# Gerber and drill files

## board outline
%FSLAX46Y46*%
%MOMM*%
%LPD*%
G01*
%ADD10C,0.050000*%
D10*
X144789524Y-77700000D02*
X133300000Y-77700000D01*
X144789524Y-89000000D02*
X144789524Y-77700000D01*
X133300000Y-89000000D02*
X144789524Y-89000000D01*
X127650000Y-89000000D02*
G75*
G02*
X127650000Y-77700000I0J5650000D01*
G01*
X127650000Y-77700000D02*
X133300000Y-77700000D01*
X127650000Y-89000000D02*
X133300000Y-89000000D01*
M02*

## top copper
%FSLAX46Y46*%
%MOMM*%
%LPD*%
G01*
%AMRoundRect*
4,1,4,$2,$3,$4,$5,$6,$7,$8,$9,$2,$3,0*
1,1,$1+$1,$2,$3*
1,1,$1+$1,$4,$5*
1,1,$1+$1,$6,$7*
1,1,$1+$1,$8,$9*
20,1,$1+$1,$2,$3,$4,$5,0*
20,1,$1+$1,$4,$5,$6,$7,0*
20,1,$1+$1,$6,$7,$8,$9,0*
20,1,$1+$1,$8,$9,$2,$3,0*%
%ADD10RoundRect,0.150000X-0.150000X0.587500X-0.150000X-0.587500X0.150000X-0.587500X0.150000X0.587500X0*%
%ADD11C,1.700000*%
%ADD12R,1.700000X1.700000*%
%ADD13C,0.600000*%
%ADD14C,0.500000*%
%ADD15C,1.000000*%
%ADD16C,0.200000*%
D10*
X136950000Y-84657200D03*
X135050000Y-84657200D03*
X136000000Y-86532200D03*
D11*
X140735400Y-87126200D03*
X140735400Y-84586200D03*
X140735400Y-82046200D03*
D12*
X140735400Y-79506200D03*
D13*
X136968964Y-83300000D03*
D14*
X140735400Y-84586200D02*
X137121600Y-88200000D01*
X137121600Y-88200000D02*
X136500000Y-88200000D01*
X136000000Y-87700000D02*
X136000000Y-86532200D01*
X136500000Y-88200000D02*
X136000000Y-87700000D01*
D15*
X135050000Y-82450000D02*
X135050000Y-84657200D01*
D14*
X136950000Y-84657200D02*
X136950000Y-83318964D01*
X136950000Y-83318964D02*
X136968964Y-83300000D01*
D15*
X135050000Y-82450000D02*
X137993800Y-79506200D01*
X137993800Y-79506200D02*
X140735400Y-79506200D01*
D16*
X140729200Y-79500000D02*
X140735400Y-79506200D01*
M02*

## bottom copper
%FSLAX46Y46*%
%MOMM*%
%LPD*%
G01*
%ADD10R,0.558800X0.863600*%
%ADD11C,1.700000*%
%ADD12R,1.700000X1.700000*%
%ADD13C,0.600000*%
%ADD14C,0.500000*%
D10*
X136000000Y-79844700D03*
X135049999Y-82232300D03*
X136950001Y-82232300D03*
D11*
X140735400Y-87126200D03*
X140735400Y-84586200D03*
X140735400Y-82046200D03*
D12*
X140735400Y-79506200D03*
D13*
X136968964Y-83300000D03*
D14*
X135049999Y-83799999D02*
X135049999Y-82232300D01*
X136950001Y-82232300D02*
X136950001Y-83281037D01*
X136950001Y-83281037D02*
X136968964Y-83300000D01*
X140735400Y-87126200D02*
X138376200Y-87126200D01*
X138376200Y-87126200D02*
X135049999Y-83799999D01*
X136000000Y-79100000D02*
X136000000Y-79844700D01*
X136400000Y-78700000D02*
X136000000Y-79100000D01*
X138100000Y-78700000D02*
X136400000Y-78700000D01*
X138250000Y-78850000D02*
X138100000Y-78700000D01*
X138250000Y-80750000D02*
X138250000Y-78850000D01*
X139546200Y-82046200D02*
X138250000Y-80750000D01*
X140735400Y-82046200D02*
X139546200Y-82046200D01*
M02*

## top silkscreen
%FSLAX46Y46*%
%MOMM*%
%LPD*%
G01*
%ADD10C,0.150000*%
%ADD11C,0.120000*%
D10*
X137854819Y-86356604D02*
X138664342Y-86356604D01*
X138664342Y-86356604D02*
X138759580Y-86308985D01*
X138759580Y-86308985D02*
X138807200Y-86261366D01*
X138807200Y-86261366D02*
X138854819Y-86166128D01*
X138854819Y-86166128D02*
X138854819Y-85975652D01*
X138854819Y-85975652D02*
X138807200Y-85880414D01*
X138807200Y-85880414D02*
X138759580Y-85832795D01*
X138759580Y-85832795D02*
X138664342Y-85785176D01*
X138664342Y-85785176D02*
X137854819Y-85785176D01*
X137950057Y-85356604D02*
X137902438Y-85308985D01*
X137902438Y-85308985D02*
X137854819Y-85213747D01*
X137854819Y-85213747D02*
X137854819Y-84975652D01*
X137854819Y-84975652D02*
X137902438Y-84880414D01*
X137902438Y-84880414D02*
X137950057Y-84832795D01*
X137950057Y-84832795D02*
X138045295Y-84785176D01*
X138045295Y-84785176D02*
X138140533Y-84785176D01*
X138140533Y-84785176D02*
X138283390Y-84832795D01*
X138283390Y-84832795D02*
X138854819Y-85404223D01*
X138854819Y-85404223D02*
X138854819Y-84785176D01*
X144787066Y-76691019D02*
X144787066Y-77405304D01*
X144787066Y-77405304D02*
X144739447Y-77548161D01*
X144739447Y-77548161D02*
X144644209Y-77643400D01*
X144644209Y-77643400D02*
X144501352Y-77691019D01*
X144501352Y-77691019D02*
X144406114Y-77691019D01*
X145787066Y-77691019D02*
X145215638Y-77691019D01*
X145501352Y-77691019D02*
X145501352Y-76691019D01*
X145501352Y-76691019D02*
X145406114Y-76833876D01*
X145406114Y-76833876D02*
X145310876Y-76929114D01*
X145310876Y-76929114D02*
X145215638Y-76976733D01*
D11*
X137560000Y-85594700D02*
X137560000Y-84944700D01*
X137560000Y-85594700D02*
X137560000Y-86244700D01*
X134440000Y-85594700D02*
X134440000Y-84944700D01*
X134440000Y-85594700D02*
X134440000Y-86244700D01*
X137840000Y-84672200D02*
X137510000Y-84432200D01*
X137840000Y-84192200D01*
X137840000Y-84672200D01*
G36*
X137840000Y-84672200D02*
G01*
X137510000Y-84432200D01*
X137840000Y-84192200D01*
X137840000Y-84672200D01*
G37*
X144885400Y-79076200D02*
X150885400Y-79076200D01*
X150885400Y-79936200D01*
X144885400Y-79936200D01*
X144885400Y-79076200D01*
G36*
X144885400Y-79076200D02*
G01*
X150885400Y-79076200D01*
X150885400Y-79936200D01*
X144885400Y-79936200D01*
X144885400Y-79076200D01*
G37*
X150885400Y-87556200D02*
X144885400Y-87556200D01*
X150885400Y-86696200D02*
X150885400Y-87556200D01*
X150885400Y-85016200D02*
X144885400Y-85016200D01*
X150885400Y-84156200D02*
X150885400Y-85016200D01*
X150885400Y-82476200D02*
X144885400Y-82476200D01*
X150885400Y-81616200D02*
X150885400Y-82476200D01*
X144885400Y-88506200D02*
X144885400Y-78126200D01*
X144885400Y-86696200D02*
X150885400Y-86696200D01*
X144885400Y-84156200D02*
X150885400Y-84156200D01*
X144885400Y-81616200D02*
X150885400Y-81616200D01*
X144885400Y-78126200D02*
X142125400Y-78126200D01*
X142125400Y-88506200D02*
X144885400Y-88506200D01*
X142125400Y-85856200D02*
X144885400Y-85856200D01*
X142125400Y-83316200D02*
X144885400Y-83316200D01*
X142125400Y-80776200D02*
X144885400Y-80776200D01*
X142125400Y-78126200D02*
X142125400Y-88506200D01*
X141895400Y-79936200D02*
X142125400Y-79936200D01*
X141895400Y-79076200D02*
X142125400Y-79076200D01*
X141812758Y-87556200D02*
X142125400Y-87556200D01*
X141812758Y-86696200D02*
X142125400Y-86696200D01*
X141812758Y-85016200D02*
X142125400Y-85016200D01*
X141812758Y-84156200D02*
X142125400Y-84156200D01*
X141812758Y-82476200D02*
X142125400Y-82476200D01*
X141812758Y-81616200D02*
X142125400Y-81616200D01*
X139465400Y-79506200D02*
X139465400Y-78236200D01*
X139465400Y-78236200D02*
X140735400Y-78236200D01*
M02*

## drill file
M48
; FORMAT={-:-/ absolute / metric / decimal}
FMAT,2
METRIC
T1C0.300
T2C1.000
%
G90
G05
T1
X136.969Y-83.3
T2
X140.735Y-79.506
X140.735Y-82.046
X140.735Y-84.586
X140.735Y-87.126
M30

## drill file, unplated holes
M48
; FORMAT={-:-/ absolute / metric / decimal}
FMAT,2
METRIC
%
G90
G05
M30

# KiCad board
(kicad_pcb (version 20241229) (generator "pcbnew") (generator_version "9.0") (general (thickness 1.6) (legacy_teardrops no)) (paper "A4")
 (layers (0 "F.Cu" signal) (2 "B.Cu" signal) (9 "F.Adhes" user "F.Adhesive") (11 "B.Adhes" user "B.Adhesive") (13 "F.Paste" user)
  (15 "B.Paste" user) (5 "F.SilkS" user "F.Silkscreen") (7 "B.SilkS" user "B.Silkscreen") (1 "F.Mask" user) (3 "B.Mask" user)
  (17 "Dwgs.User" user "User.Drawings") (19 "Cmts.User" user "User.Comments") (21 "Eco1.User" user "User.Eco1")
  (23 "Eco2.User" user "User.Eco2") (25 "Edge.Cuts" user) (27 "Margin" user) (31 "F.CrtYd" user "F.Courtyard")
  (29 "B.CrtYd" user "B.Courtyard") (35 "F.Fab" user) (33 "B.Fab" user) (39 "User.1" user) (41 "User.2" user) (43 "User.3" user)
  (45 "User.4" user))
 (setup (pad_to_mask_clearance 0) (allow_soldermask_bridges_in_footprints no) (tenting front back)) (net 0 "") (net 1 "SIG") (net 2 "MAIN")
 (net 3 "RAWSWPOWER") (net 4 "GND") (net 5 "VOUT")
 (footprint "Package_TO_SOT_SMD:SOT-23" (layer "F.Cu") (at 136 85.5947 -90)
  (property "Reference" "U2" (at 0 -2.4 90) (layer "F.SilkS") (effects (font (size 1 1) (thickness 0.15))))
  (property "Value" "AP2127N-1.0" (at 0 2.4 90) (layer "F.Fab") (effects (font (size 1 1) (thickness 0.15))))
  (fp_line (start 0 1.56) (end -0.65 1.56) (stroke (width 0.12) (type solid)) (layer "F.SilkS"))
  (fp_line (start 0 1.56) (end 0.65 1.56) (stroke (width 0.12) (type solid)) (layer "F.SilkS"))
  (fp_line (start 0 -1.56) (end -0.65 -1.56) (stroke (width 0.12) (type solid)) (layer "F.SilkS"))
  (fp_line (start 0 -1.56) (end 0.65 -1.56) (stroke (width 0.12) (type solid)) (layer "F.SilkS"))
  (fp_poly (pts (xy -1.1625 -1.51) (xy -1.4025 -1.84) (xy -0.9225 -1.84)) (stroke (width 0.12) (type solid)) (fill yes) (layer "F.SilkS"))
  (pad "1" smd roundrect (at -0.9375 -0.95 270) (size 1.475 0.6) (layers "F.Cu" "F.Mask" "F.Paste") (roundrect_rratio 0.25) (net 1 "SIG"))
  (pad "2" smd roundrect (at -0.9375 0.95 270) (size 1.475 0.6) (layers "F.Cu" "F.Mask" "F.Paste") (roundrect_rratio 0.25) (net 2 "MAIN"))
  (pad "3" smd roundrect (at 0.9375 0 270) (size 1.475 0.6) (layers "F.Cu" "F.Mask" "F.Paste") (roundrect_rratio 0.25) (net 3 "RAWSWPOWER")))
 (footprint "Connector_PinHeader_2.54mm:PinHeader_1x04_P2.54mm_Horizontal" (layer "F.Cu") (at 140.7354 79.5062)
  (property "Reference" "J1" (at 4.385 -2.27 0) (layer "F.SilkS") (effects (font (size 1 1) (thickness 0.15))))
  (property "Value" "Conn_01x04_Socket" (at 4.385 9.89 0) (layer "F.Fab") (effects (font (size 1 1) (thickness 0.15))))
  (fp_line (start -1.27 -1.27) (end 0 -1.27) (stroke (width 0.12) (type solid)) (layer "F.SilkS"))
  (fp_line (start -1.27 0) (end -1.27 -1.27) (stroke (width 0.12) (type solid)) (layer "F.SilkS"))
  (fp_line (start 1.077358 2.11) (end 1.39 2.11) (stroke (width 0.12) (type solid)) (layer "F.SilkS"))
  (fp_line (start 1.077358 2.97) (end 1.39 2.97) (stroke (width 0.12) (type solid)) (layer "F.SilkS"))
  (fp_line (start 1.077358 4.65) (end 1.39 4.65) (stroke (width 0.12) (type solid)) (layer "F.SilkS"))
  (fp_line (start 1.077358 5.51) (end 1.39 5.51) (stroke (width 0.12) (type solid)) (layer "F.SilkS"))
  (fp_line (start 1.077358 7.19) (end 1.39 7.19) (stroke (width 0.12) (type solid)) (layer "F.SilkS"))
  (fp_line (start 1.077358 8.05) (end 1.39 8.05) (stroke (width 0.12) (type solid)) (layer "F.SilkS"))
  (fp_line (start 1.16 -0.43) (end 1.39 -0.43) (stroke (width 0.12) (type solid)) (layer "F.SilkS"))
  (fp_line (start 1.16 0.43) (end 1.39 0.43) (stroke (width 0.12) (type solid)) (layer "F.SilkS"))
  (fp_line (start 1.39 -1.38) (end 1.39 9) (stroke (width 0.12) (type solid)) (layer "F.SilkS"))
  (fp_line (start 1.39 1.27) (end 4.15 1.27) (stroke (width 0.12) (type solid)) (layer "F.SilkS"))
  (fp_line (start 1.39 3.81) (end 4.15 3.81) (stroke (width 0.12) (type solid)) (layer "F.SilkS"))
  (fp_line (start 1.39 6.35) (end 4.15 6.35) (stroke (width 0.12) (type solid)) (layer "F.SilkS"))
  (fp_line (start 1.39 9) (end 4.15 9) (stroke (width 0.12) (type solid)) (layer "F.SilkS"))
  (fp_line (start 4.15 -1.38) (end 1.39 -1.38) (stroke (width 0.12) (type solid)) (layer "F.SilkS"))
  (fp_line (start 4.15 2.11) (end 10.15 2.11) (stroke (width 0.12) (type solid)) (layer "F.SilkS"))
  (fp_line (start 4.15 4.65) (end 10.15 4.65) (stroke (width 0.12) (type solid)) (layer "F.SilkS"))
  (fp_line (start 4.15 7.19) (end 10.15 7.19) (stroke (width 0.12) (type solid)) (layer "F.SilkS"))
  (fp_line (start 4.15 9) (end 4.15 -1.38) (stroke (width 0.12) (type solid)) (layer "F.SilkS"))
  (fp_line (start 10.15 2.11) (end 10.15 2.97) (stroke (width 0.12) (type solid)) (layer "F.SilkS"))
  (fp_line (start 10.15 2.97) (end 4.15 2.97) (stroke (width 0.12) (type solid)) (layer "F.SilkS"))
  (fp_line (start 10.15 4.65) (end 10.15 5.51) (stroke (width 0.12) (type solid)) (layer "F.SilkS"))
  (fp_line (start 10.15 5.51) (end 4.15 5.51) (stroke (width 0.12) (type solid)) (layer "F.SilkS"))
  (fp_line (start 10.15 7.19) (end 10.15 8.05) (stroke (width 0.12) (type solid)) (layer "F.SilkS"))
  (fp_line (start 10.15 8.05) (end 4.15 8.05) (stroke (width 0.12) (type solid)) (layer "F.SilkS"))
  (fp_rect (start 4.15 -0.43) (end 10.15 0.43) (stroke (width 0.12) (type solid)) (fill yes) (layer "F.SilkS"))
  (pad "1" thru_hole rect (at 0 0) (size 1.7 1.7) (drill 1) (layers "*.Cu" "*.Mask") (remove_unused_layers no) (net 2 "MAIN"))
  (pad "2" thru_hole circle (at 0 2.54) (size 1.7 1.7) (drill 1) (layers "*.Cu" "*.Mask") (remove_unused_layers no) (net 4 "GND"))
  (pad "3" thru_hole circle (at 0 5.08) (size 1.7 1.7) (drill 1) (layers "*.Cu" "*.Mask") (remove_unused_layers no) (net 3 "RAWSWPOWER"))
  (pad "4" thru_hole circle (at 0 7.62) (size 1.7 1.7) (drill 1) (layers "*.Cu" "*.Mask") (remove_unused_layers no) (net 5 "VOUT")))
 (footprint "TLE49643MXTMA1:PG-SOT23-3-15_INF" (layer "B.Cu") (at 136 81.0385 90)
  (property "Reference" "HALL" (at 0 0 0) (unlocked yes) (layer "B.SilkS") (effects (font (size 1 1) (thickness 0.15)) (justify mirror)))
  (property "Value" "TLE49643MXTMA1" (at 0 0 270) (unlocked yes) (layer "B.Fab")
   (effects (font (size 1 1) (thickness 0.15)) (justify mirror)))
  (pad "1" smd rect (at -1.1938 0.950001 90) (size 0.8636 0.5588) (layers "B.Cu" "B.Mask" "B.Paste") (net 1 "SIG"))
  (pad "2" smd rect (at -1.1938 -0.950001 90) (size 0.8636 0.5588) (layers "B.Cu" "B.Mask" "B.Paste") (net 5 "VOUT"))
  (pad "3" smd rect (at 1.1938 0 90) (size 0.8636 0.5588) (layers "B.Cu" "B.Mask" "B.Paste") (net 4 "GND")))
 (gr_line (start 144.789524 89) (end 144.789524 77.7) (stroke (width 0.05) (type default)) (layer "Edge.Cuts"))
 (gr_line (start 127.65 77.7) (end 133.3 77.7) (stroke (width 0.05) (type default)) (layer "Edge.Cuts"))
 (gr_line (start 127.65 89) (end 133.3 89) (stroke (width 0.05) (type default)) (layer "Edge.Cuts"))
 (gr_line (start 133.3 89) (end 144.789524 89) (stroke (width 0.05) (type default)) (layer "Edge.Cuts"))
 (gr_line (start 144.789524 77.7) (end 133.3 77.7) (stroke (width 0.05) (type default)) (layer "Edge.Cuts"))
 (gr_arc (start 127.65 89) (mid 122 83.35) (end 127.65 77.7) (stroke (width 0.05) (type default)) (layer "Edge.Cuts"))
 (segment (start 138.25 78.85) (end 138.1 78.7) (width 0.5) (layer "B.Cu") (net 4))
 (segment (start 139.5462 82.0462) (end 138.25 80.75) (width 0.5) (layer "B.Cu") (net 4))
 (segment (start 136.4 78.7) (end 136 79.1) (width 0.5) (layer "B.Cu") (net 4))
 (segment (start 138.1 78.7) (end 136.4 78.7) (width 0.5) (layer "B.Cu") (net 4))
 (segment (start 136 79.1) (end 136 79.8447) (width 0.5) (layer "B.Cu") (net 4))
 (segment (start 140.7354 82.0462) (end 139.5462 82.0462) (width 0.5) (layer "B.Cu") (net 4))
 (segment (start 138.25 80.75) (end 138.25 78.85) (width 0.5) (layer "B.Cu") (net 4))
 (segment (start 135.049999 83.799999) (end 135.049999 82.2323) (width 0.5) (layer "B.Cu") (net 5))
 (segment (start 138.3762 87.1262) (end 135.049999 83.799999) (width 0.5) (layer "B.Cu") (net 5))
 (segment (start 140.7354 87.1262) (end 138.3762 87.1262) (width 0.5) (layer "B.Cu") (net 5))
 (segment (start 140.7354 84.5862) (end 137.1216 88.2) (width 0.5) (layer "F.Cu") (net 3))
 (segment (start 136 87.7) (end 136 86.5322) (width 0.5) (layer "F.Cu") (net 3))
 (segment (start 137.1216 88.2) (end 136.5 88.2) (width 0.5) (layer "F.Cu") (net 3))
 (segment (start 136.5 88.2) (end 136 87.7) (width 0.5) (layer "F.Cu") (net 3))
 (segment (start 135.05 82.45) (end 135.05 84.6572) (width 1) (layer "F.Cu") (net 2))
 (segment (start 135.05 82.45) (end 137.9938 79.5062) (width 1) (layer "F.Cu") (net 2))
 (segment (start 140.7292 79.5) (end 140.7354 79.5062) (width 0.2) (layer "F.Cu") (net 2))
 (segment (start 137.9938 79.5062) (end 140.7354 79.5062) (width 1) (layer "F.Cu") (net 2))
 (segment (start 136.95 83.318964) (end 136.968964 83.3) (width 0.5) (layer "F.Cu") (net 1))
 (segment (start 136.95 84.6572) (end 136.95 83.318964) (width 0.5) (layer "F.Cu") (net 1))
 (via (at 136.968964 83.3) (size 0.6) (drill 0.3) (layers "F.Cu" "B.Cu") (free yes) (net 1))
 (segment (start 136.950001 82.2323) (end 136.950001 83.281037) (width 0.5) (layer "B.Cu") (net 1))
 (segment (start 136.950001 83.281037) (end 136.968964 83.3) (width 0.5) (layer "B.Cu") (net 1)))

